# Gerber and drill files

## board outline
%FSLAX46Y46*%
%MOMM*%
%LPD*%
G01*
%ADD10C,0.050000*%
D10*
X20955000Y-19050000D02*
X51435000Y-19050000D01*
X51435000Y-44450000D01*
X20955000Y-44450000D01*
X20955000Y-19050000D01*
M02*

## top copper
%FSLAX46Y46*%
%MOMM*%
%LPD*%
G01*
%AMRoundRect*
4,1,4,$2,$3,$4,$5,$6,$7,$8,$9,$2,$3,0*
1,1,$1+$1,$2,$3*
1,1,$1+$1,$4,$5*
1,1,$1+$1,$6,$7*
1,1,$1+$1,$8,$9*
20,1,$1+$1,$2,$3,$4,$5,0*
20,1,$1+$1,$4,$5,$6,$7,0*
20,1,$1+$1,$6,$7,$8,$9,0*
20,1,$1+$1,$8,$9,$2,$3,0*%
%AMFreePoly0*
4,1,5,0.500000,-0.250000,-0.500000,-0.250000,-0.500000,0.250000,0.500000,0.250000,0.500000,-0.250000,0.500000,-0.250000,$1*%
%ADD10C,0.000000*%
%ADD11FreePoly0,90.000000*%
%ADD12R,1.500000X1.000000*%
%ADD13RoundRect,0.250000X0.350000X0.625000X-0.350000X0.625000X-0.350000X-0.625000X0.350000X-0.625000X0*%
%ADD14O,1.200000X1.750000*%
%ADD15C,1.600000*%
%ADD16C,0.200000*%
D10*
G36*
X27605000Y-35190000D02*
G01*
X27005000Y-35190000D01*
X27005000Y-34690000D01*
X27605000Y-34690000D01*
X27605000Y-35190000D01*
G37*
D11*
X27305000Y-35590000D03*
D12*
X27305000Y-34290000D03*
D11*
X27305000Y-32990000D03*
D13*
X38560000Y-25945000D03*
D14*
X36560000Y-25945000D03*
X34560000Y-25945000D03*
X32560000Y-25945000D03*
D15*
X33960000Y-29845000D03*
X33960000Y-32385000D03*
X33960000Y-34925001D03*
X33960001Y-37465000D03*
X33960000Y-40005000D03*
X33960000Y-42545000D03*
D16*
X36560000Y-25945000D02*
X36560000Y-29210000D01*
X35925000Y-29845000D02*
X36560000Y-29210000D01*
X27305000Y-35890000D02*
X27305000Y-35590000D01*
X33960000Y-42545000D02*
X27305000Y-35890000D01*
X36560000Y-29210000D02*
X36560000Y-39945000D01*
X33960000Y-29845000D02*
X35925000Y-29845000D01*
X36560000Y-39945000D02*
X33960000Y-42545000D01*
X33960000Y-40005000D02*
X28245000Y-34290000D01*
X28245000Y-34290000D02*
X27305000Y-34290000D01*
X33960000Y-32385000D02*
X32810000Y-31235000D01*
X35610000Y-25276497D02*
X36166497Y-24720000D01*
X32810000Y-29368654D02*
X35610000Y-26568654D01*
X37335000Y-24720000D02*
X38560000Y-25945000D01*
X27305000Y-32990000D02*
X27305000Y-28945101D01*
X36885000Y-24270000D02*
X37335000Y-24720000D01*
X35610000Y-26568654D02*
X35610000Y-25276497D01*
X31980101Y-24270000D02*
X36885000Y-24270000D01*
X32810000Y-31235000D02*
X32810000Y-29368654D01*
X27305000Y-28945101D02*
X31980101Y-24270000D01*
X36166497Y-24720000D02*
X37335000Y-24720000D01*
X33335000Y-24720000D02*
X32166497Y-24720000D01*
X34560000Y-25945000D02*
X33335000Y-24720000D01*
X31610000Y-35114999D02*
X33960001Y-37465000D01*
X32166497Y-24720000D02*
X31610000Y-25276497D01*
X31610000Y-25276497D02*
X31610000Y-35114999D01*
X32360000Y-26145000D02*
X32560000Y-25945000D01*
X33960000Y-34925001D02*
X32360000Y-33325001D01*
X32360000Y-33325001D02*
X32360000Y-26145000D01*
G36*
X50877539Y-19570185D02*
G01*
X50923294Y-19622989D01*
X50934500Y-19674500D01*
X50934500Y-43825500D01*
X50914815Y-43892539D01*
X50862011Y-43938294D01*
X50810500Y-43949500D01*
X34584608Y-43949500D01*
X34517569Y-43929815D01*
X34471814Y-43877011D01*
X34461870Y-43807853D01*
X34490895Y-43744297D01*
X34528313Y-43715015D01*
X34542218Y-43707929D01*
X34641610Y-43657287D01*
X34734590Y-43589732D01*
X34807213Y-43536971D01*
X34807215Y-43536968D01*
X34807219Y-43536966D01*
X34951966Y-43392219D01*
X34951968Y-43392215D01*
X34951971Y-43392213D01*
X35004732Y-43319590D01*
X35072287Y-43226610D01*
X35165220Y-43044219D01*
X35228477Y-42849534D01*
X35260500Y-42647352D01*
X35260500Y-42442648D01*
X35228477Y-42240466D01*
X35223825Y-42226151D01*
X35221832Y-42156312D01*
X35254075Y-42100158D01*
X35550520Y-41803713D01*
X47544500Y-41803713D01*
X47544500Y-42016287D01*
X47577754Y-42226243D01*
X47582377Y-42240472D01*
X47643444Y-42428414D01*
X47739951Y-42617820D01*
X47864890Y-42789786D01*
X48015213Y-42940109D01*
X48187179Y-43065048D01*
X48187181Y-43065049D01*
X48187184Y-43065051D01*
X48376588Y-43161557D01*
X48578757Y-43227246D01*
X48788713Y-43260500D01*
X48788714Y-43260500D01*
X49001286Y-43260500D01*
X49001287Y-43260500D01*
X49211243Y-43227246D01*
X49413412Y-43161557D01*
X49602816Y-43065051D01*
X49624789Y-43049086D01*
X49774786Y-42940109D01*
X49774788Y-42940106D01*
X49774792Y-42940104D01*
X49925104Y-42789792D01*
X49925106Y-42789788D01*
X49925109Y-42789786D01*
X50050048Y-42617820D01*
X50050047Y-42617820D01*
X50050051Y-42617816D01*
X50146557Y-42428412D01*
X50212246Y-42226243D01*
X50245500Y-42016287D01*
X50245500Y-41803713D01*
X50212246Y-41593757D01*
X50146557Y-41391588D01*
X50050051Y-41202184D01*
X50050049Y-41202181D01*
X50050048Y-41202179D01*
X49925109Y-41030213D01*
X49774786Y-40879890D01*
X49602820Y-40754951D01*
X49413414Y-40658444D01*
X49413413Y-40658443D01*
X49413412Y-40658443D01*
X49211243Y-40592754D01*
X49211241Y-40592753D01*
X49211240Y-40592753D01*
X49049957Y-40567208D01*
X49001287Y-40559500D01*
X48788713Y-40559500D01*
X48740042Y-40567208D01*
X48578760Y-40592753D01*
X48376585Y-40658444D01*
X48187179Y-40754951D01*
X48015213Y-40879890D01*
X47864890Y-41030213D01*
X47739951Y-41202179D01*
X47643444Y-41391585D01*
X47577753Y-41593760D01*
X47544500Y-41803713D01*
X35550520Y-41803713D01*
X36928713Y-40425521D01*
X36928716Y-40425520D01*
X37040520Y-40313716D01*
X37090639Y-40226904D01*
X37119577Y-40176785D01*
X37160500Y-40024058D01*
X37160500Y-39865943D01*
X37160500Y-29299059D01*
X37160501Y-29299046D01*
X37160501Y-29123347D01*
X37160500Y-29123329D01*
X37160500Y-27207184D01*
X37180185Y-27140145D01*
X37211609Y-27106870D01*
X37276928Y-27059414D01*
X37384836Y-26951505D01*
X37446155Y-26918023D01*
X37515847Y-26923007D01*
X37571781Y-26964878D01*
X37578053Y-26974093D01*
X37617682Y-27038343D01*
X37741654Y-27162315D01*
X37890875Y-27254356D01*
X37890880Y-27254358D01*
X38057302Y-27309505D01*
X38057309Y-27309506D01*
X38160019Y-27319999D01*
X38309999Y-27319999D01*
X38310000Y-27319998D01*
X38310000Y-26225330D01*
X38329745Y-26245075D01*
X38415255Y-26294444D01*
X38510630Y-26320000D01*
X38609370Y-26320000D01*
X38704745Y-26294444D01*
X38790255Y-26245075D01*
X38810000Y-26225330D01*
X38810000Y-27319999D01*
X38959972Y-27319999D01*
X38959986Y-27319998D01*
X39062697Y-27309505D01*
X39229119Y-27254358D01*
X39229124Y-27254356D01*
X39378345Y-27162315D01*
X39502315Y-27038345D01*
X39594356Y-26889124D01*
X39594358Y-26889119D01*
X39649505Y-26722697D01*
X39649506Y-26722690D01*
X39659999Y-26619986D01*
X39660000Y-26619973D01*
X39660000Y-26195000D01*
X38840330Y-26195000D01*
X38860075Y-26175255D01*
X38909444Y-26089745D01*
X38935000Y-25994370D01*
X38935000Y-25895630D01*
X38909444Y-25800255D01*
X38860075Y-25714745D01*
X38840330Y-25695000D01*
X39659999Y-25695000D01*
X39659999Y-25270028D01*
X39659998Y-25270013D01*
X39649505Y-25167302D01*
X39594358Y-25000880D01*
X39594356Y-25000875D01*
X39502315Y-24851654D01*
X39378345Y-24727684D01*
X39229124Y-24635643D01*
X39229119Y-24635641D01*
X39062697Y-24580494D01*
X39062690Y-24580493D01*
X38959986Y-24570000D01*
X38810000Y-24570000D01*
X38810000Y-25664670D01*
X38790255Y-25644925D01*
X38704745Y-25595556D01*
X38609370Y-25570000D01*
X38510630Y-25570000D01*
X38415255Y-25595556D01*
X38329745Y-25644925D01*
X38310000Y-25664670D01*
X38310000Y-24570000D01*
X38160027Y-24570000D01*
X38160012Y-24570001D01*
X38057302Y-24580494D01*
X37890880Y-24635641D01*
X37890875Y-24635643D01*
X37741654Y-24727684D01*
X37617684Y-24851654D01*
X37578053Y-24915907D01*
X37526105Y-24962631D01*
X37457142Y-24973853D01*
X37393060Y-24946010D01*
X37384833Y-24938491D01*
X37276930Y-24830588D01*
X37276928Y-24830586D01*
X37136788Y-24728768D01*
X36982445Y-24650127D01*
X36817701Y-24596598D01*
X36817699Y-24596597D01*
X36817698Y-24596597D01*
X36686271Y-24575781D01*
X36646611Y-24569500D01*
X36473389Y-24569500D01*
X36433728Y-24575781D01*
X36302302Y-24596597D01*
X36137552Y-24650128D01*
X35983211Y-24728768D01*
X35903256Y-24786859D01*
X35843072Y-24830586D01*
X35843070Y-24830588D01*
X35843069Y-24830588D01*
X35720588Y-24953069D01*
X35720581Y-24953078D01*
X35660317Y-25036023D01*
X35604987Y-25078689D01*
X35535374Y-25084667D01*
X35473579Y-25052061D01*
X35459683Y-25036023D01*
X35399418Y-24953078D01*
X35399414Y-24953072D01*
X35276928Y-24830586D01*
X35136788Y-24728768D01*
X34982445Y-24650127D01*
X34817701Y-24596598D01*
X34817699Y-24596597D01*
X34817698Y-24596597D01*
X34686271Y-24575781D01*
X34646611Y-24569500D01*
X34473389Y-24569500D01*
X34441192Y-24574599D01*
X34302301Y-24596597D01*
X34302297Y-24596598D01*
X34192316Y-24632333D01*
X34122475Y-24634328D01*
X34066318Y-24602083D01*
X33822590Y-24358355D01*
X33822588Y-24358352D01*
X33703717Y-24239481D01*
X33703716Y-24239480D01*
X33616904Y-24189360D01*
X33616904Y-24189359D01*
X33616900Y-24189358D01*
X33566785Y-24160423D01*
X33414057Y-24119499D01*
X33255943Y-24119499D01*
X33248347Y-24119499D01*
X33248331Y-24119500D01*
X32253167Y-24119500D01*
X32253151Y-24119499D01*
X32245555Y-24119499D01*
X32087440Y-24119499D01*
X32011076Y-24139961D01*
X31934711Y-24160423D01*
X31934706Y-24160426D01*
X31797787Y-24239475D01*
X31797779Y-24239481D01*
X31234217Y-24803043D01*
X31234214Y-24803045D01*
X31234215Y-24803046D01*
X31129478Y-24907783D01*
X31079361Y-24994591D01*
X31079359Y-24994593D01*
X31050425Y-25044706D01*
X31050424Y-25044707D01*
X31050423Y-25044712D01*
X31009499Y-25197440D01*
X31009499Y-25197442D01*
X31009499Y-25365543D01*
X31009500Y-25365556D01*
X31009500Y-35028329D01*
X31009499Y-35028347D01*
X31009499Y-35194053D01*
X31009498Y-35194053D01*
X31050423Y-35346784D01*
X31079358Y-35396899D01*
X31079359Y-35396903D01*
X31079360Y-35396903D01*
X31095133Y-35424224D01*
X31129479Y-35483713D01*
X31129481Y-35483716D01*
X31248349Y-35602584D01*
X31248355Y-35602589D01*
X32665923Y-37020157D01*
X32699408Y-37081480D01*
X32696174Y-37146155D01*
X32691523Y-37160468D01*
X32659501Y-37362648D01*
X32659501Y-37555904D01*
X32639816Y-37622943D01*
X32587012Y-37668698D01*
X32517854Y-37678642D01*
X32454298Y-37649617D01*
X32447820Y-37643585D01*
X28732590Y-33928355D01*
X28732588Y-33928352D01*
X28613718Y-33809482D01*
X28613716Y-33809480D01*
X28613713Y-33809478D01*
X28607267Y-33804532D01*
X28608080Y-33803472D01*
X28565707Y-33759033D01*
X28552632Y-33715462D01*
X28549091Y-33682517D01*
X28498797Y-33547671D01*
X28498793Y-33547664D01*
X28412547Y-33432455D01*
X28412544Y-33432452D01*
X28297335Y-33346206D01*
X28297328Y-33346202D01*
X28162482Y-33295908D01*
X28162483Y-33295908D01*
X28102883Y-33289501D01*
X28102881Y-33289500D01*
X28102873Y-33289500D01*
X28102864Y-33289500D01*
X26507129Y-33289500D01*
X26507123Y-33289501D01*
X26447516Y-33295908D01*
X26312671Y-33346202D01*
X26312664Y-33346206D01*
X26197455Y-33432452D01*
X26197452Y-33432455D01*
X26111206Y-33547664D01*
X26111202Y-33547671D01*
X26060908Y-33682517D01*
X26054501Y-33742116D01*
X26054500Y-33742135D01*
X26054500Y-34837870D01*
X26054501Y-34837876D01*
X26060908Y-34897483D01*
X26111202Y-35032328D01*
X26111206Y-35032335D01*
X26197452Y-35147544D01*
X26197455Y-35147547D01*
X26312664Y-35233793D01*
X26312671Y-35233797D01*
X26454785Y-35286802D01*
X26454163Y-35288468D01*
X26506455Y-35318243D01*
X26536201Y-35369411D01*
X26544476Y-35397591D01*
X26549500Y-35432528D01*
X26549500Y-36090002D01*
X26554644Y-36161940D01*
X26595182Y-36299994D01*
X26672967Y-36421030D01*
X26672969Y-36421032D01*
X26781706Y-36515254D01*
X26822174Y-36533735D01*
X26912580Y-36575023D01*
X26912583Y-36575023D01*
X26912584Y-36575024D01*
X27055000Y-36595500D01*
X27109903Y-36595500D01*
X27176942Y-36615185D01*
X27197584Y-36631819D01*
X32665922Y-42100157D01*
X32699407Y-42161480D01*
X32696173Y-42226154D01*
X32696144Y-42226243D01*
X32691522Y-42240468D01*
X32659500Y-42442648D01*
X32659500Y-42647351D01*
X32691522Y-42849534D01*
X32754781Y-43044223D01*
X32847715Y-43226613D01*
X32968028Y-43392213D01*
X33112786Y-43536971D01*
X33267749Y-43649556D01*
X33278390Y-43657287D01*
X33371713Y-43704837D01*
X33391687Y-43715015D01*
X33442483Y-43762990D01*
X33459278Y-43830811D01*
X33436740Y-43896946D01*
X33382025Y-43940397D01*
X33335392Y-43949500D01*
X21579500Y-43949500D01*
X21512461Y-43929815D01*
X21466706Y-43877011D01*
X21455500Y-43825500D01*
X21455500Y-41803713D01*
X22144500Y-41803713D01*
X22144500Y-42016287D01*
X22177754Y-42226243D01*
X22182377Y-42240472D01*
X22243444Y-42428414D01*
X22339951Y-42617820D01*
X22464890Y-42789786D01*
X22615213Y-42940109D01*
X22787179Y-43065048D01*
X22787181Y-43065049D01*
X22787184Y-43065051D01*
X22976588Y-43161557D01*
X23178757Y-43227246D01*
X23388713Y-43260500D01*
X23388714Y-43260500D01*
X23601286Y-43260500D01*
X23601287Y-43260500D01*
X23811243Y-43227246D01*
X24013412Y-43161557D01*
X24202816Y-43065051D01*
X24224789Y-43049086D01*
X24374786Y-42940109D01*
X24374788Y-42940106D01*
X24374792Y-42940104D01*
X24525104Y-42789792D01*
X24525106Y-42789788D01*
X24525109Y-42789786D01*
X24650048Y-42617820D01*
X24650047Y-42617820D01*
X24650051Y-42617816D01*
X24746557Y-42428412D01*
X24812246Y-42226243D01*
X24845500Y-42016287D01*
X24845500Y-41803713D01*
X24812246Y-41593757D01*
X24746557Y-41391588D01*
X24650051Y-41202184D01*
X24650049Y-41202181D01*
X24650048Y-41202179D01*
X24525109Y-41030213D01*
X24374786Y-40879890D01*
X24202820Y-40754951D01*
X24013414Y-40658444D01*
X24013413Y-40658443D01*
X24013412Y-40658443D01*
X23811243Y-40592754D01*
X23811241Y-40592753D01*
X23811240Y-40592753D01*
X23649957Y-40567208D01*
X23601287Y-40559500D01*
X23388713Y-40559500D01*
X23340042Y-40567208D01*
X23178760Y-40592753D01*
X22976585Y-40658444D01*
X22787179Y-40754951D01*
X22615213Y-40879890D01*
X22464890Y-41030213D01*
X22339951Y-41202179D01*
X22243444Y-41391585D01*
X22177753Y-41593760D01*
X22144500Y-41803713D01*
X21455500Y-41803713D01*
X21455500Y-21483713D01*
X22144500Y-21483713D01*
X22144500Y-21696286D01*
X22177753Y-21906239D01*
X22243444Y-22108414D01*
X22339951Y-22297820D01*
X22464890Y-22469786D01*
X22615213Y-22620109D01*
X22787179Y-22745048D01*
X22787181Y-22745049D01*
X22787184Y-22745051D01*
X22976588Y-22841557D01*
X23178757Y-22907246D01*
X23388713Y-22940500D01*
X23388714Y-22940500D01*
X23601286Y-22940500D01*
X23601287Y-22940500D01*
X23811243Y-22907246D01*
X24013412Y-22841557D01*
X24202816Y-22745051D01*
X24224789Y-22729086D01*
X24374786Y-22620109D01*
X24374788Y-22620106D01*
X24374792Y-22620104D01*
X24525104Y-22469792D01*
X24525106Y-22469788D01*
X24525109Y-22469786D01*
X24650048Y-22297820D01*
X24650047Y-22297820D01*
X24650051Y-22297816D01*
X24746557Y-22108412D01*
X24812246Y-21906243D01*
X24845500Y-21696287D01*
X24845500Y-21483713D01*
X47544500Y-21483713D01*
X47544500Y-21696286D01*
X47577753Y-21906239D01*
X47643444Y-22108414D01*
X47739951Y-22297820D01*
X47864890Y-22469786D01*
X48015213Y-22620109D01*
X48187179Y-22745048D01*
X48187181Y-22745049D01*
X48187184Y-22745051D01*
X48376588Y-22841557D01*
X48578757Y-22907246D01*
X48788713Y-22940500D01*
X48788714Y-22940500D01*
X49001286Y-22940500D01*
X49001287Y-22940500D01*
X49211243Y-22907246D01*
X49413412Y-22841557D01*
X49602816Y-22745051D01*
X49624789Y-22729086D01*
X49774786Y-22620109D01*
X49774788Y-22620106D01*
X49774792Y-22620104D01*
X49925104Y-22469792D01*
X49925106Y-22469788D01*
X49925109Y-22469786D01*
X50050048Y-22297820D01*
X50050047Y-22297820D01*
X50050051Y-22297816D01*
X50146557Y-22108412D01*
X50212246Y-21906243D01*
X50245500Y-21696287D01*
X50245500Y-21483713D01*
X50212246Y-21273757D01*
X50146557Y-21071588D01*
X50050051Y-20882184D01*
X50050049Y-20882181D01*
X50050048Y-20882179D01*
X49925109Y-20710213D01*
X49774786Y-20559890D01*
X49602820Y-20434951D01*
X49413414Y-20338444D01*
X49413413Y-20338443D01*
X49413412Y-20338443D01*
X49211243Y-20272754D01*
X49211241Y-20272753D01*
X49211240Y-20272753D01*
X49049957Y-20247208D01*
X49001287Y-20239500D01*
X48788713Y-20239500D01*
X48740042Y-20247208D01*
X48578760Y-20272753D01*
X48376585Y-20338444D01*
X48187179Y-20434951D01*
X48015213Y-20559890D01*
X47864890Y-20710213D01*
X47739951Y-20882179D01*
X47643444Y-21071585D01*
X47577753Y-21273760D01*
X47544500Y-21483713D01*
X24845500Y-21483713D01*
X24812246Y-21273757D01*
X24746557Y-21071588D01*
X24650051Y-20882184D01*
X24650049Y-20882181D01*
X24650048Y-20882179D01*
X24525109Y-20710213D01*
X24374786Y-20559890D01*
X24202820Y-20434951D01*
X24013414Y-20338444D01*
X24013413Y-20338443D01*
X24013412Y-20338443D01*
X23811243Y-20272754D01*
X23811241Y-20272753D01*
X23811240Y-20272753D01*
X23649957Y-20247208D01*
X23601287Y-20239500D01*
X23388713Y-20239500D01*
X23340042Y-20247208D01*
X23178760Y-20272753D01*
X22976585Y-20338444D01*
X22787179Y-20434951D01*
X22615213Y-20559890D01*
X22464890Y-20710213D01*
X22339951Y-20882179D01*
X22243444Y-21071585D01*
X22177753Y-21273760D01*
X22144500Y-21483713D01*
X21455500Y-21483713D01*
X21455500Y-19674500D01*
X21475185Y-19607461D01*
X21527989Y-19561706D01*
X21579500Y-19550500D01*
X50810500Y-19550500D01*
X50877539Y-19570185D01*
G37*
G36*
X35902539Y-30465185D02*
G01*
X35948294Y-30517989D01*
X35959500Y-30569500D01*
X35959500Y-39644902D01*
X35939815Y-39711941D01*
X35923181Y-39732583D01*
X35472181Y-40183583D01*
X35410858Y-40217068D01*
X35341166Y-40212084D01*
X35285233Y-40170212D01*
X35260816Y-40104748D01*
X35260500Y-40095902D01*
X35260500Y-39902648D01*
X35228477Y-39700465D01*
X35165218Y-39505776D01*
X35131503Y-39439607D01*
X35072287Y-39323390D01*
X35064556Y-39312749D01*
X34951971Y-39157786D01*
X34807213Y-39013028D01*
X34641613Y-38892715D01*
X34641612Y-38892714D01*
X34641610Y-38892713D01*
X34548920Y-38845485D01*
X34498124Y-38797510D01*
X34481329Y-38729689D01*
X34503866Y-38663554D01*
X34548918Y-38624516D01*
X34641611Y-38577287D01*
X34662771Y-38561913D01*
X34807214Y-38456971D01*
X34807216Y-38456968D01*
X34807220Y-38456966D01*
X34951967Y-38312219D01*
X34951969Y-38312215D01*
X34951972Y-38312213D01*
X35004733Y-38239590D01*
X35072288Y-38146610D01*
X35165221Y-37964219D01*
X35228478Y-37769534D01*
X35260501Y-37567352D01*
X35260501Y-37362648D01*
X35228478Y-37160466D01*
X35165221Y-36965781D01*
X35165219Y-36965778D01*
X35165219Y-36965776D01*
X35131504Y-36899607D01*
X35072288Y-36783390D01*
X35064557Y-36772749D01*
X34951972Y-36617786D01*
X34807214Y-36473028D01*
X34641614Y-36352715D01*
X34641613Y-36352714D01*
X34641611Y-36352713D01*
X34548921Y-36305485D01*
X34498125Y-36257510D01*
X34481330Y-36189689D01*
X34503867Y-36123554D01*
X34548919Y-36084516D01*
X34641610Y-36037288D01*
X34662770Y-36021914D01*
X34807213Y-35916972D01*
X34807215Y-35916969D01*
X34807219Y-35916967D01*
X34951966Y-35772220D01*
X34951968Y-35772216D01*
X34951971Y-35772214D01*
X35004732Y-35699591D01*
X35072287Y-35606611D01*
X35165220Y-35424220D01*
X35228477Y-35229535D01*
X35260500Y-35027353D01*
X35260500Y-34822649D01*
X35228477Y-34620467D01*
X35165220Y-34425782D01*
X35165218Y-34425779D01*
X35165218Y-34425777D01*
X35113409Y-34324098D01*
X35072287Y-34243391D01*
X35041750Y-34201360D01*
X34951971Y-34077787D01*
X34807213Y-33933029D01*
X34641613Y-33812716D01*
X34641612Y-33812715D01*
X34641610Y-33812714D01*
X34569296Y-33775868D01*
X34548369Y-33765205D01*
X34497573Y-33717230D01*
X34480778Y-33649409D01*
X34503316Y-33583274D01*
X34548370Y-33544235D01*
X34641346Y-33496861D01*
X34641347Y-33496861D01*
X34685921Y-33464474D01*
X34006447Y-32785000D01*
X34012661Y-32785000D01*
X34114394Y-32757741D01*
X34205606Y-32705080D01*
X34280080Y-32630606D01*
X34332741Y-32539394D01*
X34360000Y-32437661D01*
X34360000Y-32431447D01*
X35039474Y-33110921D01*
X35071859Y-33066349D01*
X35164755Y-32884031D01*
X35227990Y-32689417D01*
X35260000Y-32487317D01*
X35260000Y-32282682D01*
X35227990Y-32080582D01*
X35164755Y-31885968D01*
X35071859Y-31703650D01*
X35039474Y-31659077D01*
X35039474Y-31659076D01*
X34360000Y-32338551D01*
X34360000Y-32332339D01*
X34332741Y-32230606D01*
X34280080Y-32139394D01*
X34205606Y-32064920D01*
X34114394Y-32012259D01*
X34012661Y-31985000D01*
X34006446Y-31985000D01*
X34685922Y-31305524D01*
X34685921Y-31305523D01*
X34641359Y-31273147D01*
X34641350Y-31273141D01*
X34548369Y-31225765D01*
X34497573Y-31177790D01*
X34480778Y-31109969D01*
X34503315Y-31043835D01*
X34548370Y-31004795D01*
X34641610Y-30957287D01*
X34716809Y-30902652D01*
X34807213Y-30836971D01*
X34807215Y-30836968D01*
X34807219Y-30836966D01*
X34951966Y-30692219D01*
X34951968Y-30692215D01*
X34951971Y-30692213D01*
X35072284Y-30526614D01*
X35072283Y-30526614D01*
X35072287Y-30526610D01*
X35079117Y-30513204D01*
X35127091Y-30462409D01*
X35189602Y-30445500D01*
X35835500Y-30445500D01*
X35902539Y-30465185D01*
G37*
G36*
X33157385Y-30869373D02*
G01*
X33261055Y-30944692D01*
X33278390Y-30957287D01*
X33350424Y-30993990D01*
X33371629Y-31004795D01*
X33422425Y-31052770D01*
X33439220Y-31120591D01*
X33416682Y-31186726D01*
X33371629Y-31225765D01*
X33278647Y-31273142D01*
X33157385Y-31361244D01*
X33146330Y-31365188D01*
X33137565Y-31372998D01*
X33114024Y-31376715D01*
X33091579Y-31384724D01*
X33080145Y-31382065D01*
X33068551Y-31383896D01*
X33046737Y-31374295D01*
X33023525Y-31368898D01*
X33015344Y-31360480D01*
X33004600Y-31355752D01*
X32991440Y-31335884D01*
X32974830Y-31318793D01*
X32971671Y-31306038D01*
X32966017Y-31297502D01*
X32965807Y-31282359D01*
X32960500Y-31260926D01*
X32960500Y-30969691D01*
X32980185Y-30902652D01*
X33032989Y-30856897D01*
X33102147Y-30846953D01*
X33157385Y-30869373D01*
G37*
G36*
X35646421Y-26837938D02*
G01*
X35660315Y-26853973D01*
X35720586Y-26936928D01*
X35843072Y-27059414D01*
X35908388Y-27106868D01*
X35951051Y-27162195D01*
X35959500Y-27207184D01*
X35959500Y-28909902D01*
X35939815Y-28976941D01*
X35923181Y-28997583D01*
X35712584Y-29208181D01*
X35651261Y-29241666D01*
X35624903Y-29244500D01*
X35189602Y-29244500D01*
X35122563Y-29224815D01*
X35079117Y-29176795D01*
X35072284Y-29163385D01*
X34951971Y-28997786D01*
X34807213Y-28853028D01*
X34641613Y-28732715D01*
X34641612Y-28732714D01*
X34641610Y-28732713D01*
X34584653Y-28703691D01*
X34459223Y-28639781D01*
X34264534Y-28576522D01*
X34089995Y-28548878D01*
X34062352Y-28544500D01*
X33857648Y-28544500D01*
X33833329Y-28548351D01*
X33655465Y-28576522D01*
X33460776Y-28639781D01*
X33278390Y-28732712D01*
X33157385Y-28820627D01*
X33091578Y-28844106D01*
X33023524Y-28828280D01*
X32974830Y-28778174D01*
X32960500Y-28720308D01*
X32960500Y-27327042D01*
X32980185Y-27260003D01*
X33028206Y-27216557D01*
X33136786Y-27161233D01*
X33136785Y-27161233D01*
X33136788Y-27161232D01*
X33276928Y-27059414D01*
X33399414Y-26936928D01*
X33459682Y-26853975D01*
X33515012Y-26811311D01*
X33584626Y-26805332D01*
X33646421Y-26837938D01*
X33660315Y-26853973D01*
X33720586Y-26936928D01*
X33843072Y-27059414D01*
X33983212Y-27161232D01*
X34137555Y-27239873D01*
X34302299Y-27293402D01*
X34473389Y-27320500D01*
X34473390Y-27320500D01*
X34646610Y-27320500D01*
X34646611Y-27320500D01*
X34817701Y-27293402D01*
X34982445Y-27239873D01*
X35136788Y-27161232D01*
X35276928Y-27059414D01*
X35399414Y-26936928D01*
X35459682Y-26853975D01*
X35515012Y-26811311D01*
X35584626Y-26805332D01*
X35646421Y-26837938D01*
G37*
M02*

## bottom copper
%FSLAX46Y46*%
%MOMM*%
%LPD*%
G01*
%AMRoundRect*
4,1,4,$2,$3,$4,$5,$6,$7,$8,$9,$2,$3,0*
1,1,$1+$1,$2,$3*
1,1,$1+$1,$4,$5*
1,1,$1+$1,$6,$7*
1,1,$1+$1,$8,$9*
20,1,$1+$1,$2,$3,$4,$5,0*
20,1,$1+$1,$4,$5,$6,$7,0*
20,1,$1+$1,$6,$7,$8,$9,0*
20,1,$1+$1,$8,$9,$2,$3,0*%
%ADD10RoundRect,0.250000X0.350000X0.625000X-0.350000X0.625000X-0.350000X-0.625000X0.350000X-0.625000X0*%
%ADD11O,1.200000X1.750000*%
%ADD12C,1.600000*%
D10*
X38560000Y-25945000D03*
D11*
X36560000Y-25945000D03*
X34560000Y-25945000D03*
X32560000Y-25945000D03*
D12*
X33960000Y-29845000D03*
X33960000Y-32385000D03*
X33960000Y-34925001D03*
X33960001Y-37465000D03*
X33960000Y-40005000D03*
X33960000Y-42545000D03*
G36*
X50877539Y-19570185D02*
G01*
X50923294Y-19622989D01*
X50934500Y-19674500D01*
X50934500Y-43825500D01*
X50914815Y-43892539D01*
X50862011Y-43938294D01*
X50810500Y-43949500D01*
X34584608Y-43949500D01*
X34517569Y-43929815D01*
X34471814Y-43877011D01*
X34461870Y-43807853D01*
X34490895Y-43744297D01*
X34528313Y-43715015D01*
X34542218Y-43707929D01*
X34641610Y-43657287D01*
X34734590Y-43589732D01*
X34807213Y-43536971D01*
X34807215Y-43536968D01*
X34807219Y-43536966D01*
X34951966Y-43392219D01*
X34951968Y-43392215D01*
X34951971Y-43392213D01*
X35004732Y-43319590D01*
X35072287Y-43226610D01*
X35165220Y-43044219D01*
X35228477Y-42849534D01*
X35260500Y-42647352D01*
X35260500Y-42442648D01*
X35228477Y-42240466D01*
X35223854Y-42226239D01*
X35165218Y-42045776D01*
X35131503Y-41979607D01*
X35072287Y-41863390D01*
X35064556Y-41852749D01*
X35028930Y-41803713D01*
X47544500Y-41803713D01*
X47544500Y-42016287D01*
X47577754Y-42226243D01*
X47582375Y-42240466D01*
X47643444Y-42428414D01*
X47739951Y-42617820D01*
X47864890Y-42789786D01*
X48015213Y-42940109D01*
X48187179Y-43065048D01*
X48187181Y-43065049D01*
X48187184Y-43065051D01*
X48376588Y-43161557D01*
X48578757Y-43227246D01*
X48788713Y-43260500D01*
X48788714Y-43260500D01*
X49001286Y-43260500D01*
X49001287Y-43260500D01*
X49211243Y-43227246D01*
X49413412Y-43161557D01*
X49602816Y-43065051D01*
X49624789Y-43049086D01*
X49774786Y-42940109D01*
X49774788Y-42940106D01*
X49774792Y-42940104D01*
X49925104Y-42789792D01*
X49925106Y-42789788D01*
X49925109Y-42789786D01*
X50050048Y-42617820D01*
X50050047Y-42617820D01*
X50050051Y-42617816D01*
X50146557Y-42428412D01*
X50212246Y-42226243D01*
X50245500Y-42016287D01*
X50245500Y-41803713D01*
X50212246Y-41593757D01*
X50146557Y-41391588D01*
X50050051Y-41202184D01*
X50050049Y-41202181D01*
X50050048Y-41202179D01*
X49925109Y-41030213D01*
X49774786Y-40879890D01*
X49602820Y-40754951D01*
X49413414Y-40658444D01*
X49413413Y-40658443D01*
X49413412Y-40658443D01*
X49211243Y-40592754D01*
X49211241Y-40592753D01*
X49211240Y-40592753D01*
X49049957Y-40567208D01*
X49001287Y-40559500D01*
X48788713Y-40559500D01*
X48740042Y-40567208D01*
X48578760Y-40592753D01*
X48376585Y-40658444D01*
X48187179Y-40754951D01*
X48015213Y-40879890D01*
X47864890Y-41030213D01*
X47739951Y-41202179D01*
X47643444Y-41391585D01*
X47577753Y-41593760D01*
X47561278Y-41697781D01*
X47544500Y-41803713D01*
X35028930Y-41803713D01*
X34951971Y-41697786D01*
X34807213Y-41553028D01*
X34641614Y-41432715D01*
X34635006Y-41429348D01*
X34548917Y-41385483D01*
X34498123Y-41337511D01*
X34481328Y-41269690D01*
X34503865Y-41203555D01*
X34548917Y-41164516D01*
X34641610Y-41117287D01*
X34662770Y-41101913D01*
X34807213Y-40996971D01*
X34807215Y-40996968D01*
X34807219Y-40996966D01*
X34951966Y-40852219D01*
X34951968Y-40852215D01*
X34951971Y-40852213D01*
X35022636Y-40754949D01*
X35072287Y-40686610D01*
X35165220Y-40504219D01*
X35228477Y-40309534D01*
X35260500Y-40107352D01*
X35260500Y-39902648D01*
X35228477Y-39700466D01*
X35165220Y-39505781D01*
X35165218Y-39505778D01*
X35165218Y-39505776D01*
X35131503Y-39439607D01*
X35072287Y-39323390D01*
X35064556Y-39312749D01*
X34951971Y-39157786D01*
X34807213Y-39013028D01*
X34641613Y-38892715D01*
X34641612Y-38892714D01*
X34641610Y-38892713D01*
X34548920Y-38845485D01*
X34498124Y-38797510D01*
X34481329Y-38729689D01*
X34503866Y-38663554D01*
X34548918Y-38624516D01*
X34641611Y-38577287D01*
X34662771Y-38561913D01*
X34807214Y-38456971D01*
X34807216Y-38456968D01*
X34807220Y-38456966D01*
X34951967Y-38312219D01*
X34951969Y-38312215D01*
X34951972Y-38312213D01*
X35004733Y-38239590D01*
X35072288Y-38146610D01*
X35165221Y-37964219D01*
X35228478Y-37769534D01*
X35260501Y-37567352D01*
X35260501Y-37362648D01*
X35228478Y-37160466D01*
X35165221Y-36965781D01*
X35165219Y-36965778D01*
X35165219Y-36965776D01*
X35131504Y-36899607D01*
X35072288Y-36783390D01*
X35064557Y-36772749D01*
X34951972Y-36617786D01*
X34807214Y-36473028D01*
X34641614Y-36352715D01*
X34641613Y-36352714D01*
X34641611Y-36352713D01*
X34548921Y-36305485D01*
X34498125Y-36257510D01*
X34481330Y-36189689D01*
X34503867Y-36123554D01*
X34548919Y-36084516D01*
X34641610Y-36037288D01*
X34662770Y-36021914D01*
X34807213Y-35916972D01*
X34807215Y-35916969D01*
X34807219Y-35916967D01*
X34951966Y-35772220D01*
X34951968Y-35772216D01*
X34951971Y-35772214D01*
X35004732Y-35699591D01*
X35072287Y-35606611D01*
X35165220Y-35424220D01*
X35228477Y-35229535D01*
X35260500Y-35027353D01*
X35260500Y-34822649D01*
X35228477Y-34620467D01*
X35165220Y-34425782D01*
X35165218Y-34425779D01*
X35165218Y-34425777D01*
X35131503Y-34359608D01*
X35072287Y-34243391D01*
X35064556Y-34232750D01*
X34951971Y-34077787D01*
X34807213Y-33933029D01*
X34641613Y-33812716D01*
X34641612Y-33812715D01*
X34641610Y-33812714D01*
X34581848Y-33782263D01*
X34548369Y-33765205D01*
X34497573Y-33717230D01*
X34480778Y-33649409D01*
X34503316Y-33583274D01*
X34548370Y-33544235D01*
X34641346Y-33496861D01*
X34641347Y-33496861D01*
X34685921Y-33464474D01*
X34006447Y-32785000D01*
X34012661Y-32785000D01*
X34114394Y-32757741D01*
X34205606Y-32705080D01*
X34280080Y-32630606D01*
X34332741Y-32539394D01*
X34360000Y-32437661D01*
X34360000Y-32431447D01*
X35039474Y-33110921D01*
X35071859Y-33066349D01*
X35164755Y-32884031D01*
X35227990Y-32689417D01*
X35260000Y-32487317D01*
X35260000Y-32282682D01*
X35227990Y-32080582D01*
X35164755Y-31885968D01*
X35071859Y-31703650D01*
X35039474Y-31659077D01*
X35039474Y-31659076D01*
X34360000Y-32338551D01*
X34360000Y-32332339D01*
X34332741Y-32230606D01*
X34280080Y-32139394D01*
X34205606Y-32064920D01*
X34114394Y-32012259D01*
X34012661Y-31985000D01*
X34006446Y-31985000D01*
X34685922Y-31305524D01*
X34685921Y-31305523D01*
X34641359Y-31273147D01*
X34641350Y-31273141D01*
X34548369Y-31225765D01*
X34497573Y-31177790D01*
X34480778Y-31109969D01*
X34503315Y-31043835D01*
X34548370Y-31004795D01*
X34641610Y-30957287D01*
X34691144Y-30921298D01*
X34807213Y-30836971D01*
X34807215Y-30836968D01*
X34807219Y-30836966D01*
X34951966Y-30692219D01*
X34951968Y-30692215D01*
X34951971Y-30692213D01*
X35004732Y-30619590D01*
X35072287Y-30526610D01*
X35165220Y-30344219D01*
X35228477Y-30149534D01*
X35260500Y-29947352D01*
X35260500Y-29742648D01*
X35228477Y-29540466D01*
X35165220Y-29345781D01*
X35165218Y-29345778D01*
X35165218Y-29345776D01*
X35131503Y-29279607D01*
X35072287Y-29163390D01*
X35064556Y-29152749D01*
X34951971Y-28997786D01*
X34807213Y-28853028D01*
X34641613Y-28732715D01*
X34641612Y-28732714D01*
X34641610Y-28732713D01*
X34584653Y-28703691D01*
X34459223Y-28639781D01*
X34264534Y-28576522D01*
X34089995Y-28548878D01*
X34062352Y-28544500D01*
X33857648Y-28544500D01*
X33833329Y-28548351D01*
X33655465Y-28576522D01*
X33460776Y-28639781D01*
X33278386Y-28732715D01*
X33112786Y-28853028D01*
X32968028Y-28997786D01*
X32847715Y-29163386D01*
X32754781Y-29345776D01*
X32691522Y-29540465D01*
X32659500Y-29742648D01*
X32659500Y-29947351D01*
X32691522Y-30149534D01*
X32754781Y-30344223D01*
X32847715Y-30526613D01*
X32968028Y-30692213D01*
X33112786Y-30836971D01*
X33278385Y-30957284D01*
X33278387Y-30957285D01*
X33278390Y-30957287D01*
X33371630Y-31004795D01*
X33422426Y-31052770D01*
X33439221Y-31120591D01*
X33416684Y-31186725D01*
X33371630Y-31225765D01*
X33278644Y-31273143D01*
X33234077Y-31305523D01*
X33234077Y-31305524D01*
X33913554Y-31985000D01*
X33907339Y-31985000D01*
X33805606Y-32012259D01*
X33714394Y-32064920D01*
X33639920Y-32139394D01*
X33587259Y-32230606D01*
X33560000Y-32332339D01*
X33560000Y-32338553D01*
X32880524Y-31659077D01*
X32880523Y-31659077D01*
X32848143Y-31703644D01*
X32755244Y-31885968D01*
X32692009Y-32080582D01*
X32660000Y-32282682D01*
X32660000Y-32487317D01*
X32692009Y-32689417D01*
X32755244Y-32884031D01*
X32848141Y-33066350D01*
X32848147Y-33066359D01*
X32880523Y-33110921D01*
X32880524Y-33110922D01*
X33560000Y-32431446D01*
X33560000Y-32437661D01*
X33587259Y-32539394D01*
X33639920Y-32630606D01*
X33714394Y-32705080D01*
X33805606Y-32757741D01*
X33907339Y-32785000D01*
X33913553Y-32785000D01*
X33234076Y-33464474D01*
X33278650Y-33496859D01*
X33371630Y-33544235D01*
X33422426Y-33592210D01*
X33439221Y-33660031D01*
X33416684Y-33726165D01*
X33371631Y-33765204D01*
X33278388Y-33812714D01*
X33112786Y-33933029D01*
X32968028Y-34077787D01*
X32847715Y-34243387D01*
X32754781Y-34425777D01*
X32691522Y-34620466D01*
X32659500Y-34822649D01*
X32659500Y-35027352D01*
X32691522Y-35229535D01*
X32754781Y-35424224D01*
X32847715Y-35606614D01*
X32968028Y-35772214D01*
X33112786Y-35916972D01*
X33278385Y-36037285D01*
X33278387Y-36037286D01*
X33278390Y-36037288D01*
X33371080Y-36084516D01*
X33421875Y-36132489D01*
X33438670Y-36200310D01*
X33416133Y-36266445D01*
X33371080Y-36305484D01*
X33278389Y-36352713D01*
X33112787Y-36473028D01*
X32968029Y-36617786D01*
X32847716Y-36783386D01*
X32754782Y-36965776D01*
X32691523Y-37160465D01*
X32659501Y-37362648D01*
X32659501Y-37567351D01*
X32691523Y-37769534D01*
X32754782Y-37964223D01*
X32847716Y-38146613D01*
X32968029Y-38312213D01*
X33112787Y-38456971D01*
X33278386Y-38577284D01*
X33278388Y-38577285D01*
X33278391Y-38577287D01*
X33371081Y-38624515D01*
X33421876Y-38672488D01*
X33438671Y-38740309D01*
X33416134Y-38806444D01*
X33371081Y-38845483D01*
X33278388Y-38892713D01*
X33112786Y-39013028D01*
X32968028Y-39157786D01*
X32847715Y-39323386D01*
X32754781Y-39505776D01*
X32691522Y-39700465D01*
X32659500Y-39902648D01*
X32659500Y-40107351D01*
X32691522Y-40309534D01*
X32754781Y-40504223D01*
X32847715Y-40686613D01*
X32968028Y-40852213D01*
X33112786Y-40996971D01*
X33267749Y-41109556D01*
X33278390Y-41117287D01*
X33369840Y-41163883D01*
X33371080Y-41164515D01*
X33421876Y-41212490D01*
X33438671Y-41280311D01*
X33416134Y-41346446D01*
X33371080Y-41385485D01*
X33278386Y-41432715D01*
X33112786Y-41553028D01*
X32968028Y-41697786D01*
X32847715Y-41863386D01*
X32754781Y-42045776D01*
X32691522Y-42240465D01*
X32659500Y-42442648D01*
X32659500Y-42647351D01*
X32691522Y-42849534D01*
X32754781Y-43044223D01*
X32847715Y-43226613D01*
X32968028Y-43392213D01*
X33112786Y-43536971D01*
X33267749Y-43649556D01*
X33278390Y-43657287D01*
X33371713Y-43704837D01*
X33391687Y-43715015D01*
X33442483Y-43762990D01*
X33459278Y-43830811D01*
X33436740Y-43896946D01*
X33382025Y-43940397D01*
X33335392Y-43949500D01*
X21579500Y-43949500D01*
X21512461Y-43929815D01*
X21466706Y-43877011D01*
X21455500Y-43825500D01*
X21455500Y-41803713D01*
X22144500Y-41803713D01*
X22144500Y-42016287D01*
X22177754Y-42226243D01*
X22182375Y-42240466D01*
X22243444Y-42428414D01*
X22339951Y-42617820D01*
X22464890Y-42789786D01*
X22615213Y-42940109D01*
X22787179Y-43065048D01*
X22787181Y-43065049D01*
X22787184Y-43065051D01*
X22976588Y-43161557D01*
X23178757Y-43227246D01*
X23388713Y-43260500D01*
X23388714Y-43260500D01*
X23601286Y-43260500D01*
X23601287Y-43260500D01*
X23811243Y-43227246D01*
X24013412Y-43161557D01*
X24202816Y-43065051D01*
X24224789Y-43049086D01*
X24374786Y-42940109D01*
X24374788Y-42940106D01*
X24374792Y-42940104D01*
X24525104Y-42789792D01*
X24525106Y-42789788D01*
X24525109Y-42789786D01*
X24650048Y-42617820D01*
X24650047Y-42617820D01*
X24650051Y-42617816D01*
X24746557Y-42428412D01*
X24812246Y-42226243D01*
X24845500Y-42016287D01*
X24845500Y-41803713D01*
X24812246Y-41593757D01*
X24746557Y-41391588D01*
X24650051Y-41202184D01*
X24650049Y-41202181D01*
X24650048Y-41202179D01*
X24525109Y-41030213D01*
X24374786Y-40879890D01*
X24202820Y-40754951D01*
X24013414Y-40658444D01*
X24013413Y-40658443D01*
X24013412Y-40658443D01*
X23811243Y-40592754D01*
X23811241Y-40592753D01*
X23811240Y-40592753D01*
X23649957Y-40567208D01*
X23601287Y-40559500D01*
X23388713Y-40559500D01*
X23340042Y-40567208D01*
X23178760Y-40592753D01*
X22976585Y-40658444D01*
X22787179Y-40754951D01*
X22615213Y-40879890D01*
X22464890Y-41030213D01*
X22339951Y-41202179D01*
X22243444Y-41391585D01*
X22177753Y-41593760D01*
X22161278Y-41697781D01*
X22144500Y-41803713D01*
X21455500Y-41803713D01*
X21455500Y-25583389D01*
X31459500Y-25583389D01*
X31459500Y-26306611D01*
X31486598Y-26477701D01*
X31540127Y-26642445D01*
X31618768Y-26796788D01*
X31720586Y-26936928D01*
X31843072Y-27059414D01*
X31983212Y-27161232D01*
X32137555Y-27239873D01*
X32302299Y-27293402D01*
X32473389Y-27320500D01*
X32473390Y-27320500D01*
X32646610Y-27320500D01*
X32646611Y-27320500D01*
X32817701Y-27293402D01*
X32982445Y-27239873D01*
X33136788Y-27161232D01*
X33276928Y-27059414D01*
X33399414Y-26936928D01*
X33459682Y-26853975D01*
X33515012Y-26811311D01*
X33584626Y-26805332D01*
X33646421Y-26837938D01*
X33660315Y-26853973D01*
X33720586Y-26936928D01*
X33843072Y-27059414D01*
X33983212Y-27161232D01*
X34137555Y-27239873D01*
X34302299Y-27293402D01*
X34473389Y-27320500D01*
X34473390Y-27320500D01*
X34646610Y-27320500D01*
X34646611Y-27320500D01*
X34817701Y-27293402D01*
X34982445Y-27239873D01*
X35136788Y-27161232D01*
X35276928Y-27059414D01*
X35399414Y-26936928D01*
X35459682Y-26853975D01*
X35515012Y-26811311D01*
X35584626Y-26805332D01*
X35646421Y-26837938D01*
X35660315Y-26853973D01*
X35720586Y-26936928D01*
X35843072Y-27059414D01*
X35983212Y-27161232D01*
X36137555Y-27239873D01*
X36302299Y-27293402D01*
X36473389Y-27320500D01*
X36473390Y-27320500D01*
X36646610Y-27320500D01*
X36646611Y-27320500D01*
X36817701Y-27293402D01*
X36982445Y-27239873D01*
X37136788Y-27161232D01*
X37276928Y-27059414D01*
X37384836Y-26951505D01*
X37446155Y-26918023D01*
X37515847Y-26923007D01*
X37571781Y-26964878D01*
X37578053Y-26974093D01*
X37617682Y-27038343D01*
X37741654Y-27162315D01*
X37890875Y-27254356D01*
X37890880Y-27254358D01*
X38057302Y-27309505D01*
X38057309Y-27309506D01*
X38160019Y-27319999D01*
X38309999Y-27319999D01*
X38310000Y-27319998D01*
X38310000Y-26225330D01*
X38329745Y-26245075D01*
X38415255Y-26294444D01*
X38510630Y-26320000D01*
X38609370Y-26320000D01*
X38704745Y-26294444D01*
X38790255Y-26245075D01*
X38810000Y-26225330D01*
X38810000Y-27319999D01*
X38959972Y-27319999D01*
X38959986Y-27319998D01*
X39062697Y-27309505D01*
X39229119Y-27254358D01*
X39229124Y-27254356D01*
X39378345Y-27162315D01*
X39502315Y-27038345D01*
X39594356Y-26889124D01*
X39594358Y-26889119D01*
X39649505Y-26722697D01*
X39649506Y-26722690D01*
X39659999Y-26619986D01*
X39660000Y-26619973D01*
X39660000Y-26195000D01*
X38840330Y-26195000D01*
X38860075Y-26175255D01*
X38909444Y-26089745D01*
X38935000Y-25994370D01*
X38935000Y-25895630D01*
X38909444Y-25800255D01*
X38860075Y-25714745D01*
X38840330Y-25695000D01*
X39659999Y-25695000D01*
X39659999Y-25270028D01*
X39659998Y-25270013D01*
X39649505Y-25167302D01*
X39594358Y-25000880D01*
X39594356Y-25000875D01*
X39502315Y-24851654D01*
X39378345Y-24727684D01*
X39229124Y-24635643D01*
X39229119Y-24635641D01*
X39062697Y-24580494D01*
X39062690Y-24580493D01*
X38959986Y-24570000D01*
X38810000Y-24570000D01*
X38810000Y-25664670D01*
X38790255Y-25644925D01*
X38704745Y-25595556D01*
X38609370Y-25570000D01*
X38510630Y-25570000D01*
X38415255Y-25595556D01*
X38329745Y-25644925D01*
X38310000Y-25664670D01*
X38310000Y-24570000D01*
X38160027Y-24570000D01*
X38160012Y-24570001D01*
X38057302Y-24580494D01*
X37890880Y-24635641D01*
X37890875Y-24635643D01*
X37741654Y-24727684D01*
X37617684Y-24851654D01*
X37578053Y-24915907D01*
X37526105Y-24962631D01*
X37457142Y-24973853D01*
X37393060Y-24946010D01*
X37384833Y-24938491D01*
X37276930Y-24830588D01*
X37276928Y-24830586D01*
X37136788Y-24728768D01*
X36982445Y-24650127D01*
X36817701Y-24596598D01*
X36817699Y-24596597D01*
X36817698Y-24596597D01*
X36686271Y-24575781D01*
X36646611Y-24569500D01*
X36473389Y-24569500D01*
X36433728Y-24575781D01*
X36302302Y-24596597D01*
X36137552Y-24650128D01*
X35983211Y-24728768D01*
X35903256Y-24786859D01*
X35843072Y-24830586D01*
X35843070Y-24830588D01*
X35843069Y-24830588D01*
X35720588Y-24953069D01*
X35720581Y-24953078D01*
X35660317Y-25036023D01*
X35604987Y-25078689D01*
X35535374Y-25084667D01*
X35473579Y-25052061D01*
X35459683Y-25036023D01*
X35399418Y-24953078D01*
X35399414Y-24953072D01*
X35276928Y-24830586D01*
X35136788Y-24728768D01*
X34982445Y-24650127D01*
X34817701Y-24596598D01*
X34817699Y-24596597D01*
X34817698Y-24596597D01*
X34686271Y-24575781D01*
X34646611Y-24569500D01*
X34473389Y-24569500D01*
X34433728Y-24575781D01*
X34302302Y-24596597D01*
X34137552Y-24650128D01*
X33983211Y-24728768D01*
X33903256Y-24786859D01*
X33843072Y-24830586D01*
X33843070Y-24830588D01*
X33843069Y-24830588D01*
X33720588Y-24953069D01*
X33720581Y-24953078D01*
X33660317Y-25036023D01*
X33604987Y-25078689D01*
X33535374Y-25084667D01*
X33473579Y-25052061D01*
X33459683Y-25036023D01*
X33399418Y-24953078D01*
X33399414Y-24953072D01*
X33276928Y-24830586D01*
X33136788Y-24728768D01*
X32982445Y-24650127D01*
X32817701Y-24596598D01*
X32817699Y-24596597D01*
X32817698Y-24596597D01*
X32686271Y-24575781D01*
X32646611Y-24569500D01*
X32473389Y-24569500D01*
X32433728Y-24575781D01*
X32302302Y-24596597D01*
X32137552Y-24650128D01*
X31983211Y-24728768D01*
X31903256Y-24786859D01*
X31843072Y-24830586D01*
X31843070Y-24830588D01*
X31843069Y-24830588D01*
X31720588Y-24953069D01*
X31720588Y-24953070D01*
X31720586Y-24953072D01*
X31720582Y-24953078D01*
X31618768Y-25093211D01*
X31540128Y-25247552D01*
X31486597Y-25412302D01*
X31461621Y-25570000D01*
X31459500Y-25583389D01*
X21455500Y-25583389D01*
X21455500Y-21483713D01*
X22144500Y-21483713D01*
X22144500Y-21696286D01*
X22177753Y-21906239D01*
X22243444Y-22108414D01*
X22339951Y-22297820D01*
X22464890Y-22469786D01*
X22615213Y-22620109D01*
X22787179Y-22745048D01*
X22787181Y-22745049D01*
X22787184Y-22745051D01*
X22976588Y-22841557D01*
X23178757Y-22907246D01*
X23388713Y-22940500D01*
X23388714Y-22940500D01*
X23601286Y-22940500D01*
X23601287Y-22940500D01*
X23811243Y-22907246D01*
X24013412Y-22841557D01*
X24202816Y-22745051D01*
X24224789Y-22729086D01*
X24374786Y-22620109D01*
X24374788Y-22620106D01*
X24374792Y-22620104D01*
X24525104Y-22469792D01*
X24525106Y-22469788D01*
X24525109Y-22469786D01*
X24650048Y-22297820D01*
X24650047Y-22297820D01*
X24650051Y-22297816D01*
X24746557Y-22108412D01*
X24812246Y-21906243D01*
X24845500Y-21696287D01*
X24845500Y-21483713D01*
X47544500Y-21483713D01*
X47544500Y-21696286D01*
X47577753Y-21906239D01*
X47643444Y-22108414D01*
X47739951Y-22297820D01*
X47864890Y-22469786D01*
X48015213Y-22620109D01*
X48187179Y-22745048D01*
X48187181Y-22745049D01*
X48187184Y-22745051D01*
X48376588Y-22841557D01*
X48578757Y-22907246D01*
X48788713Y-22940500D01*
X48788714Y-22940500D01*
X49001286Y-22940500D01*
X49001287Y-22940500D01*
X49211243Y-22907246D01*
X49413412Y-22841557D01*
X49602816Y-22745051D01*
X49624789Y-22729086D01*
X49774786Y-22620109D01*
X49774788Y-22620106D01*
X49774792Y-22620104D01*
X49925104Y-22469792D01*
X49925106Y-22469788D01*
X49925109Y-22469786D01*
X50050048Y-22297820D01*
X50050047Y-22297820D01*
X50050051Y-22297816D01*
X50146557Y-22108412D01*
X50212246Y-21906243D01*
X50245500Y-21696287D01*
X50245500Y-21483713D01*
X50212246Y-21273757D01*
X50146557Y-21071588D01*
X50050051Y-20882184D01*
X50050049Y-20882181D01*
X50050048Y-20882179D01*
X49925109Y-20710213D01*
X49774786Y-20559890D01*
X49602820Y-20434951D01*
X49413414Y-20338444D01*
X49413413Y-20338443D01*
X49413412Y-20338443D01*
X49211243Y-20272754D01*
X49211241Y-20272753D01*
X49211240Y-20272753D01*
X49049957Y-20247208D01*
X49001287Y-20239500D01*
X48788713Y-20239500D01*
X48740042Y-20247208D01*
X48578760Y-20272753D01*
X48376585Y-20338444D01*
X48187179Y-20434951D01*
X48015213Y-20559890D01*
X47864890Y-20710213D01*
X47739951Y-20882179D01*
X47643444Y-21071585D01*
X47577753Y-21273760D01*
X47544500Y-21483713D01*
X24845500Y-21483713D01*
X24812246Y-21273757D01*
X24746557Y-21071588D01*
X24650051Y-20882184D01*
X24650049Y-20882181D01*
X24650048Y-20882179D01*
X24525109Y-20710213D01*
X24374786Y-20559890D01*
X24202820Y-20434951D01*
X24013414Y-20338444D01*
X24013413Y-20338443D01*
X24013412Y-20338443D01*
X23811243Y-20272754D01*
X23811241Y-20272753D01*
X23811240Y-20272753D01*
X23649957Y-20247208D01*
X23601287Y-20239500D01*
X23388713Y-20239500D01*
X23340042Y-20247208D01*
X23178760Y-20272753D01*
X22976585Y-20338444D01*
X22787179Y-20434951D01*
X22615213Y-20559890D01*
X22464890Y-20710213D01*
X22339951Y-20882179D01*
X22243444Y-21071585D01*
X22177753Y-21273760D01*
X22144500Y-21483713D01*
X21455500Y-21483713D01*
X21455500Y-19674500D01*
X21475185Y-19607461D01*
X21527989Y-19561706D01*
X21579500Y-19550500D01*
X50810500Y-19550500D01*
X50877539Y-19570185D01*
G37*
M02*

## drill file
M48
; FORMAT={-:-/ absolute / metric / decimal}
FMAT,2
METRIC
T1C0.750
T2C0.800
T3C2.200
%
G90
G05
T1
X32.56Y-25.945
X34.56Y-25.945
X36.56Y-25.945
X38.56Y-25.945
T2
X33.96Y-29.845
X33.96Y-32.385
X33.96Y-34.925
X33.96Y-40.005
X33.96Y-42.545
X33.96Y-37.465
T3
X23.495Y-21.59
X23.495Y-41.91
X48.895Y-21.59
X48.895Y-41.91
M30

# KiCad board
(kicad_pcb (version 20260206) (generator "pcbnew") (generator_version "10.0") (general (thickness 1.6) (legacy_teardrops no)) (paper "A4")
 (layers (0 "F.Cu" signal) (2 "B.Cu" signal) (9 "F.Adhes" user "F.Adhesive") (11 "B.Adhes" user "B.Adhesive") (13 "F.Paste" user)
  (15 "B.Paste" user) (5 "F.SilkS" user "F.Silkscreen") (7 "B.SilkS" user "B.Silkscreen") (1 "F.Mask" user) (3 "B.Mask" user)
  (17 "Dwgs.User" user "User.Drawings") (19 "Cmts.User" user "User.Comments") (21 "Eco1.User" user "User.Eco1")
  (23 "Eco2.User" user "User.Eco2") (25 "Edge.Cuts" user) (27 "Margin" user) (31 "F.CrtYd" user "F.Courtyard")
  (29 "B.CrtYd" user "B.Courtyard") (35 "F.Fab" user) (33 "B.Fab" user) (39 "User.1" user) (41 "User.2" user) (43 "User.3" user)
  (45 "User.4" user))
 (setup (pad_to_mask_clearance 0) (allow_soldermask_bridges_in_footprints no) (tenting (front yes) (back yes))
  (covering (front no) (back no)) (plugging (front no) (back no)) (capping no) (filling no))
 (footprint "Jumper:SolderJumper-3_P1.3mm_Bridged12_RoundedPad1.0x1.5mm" (layer "F.Cu") (at 27.305 34.29 90)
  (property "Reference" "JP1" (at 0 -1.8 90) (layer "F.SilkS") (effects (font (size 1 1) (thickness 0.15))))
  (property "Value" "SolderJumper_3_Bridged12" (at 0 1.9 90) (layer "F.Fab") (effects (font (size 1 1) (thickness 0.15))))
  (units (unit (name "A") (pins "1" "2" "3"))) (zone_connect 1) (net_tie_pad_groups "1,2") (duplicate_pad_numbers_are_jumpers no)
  (fp_poly (pts (xy -0.9 -0.3) (xy -0.4 -0.3) (xy -0.4 0.3) (xy -0.9 0.3)) (stroke (width 0) (type solid)) (fill yes) (layer "F.Cu"))
  (pad "1" smd custom (at -1.3 0 90) (size 1 0.5) (layers "F.Cu" "F.Mask") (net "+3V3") (zone_connect 2) (thermal_bridge_angle 45)
   (options (clearance outline) (anchor rect)) (primitives))
  (pad "2" smd rect (at 0 0 90) (size 1 1.5) (layers "F.Cu" "F.Mask") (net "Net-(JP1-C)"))
  (pad "3" smd custom (at 1.3 0 90) (size 1 0.5) (layers "F.Cu" "F.Mask") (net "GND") (zone_connect 2) (thermal_bridge_angle 45)
   (options (clearance outline) (anchor rect)) (primitives)))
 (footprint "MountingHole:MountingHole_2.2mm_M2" (layer "F.Cu") (at 48.895 21.59)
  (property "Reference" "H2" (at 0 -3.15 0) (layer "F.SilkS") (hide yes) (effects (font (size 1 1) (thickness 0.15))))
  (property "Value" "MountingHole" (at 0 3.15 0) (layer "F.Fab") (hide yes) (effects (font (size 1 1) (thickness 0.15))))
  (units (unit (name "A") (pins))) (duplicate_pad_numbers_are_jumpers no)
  (pad "" np_thru_hole circle (at 0 0) (size 2.2 2.2) (drill 2.2) (layers "*.Cu" "*.Mask")))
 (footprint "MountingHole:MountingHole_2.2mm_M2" (layer "F.Cu") (at 48.895 41.91)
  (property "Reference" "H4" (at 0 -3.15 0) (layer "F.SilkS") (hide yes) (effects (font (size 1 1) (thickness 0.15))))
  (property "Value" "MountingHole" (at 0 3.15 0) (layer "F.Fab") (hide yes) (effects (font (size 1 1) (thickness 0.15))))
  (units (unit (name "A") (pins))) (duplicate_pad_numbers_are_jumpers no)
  (pad "" np_thru_hole circle (at 0 0) (size 2.2 2.2) (drill 2.2) (layers "*.Cu" "*.Mask")))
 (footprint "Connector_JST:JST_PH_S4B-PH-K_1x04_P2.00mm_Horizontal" (layer "F.Cu") (at 38.56 25.945 180)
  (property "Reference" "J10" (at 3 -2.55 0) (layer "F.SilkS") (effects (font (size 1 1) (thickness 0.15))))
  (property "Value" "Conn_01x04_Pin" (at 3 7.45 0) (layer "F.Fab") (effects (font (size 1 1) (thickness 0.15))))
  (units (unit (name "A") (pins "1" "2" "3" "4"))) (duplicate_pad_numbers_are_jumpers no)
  (pad "1" thru_hole roundrect (at 0 0 180) (size 1.2 1.75) (drill 0.75) (layers "*.Cu" "*.Mask") (remove_unused_layers no)
   (roundrect_rratio 0.208333) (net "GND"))
  (pad "2" thru_hole oval (at 2 0 180) (size 1.2 1.75) (drill 0.75) (layers "*.Cu" "*.Mask") (remove_unused_layers no) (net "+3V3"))
  (pad "3" thru_hole oval (at 4 0 180) (size 1.2 1.75) (drill 0.75) (layers "*.Cu" "*.Mask") (remove_unused_layers no) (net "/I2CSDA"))
  (pad "4" thru_hole oval (at 6 0 180) (size 1.2 1.75) (drill 0.75) (layers "*.Cu" "*.Mask") (remove_unused_layers no) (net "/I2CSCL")))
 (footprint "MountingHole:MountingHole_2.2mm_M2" (layer "F.Cu") (at 23.495 21.59)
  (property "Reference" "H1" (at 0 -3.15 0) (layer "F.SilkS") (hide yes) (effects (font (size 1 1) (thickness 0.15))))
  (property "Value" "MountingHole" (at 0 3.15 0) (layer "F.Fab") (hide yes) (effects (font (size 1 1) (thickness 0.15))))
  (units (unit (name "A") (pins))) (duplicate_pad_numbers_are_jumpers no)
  (pad "" np_thru_hole circle (at 0 0) (size 2.2 2.2) (drill 2.2) (layers "*.Cu" "*.Mask")))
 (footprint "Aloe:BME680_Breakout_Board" (layer "F.Cu") (at 40.31 36.195 -90)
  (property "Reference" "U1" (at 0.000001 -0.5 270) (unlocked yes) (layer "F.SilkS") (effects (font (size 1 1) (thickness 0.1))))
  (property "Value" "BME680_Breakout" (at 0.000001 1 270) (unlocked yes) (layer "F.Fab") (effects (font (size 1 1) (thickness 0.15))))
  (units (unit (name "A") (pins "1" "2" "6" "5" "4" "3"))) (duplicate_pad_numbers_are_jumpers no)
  (pad "1" thru_hole circle (at -6.35 6.35 270) (size 1.6 1.6) (drill 0.8) (layers "*.Cu" "*.Mask") (remove_unused_layers no) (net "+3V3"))
  (pad "2" thru_hole circle (at -3.81 6.35 270) (size 1.6 1.6) (drill 0.8) (layers "*.Cu" "*.Mask") (remove_unused_layers no) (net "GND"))
  (pad "3" thru_hole circle (at -1.269999 6.35 270) (size 1.6 1.6) (drill 0.8) (layers "*.Cu" "*.Mask") (remove_unused_layers no)
   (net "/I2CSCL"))
  (pad "4" thru_hole circle (at 1.27 6.349999 270) (size 1.6 1.6) (drill 0.8) (layers "*.Cu" "*.Mask") (remove_unused_layers no)
   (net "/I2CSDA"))
  (pad "5" thru_hole circle (at 3.81 6.35 270) (size 1.6 1.6) (drill 0.8) (layers "*.Cu" "*.Mask") (remove_unused_layers no)
   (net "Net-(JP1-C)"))
  (pad "6" thru_hole circle (at 6.35 6.35 270) (size 1.6 1.6) (drill 0.8) (layers "*.Cu" "*.Mask") (remove_unused_layers no) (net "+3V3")))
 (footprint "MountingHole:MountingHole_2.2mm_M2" (layer "F.Cu") (at 23.495 41.91)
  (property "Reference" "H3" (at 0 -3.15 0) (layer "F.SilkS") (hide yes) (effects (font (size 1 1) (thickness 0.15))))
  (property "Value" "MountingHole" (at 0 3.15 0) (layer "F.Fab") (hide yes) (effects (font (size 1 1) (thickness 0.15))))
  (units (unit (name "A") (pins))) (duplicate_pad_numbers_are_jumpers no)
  (pad "" np_thru_hole circle (at 0 0) (size 2.2 2.2) (drill 2.2) (layers "*.Cu" "*.Mask")))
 (gr_rect (start 20.955 19.05) (end 51.435 44.45) (stroke (width 0.05) (type solid)) (fill no) (layer "Edge.Cuts"))
 (segment (start 36.56 25.945) (end 36.56 29.21) (width 0.2) (layer "F.Cu") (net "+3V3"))
 (segment (start 35.925 29.845) (end 36.56 29.21) (width 0.2) (layer "F.Cu") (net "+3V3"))
 (segment (start 27.305 35.89) (end 27.305 35.59) (width 0.2) (layer "F.Cu") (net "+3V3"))
 (segment (start 33.96 42.545) (end 27.305 35.89) (width 0.2) (layer "F.Cu") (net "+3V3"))
 (segment (start 36.56 29.21) (end 36.56 39.945) (width 0.2) (layer "F.Cu") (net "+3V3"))
 (segment (start 33.96 29.845) (end 35.925 29.845) (width 0.2) (layer "F.Cu") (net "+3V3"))
 (segment (start 36.56 39.945) (end 33.96 42.545) (width 0.2) (layer "F.Cu") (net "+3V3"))
 (segment (start 33.96 40.005) (end 28.245 34.29) (width 0.2) (layer "F.Cu") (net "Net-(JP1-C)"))
 (segment (start 28.245 34.29) (end 27.305 34.29) (width 0.2) (layer "F.Cu") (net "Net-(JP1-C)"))
 (segment (start 33.96 32.385) (end 32.81 31.235) (width 0.2) (layer "F.Cu") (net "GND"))
 (segment (start 35.61 25.276497) (end 36.166497 24.72) (width 0.2) (layer "F.Cu") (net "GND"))
 (segment (start 32.81 29.368654) (end 35.61 26.568654) (width 0.2) (layer "F.Cu") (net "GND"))
 (segment (start 37.335 24.72) (end 38.56 25.945) (width 0.2) (layer "F.Cu") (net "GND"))
 (segment (start 27.305 32.99) (end 27.305 28.945101) (width 0.2) (layer "F.Cu") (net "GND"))
 (segment (start 36.885 24.27) (end 37.335 24.72) (width 0.2) (layer "F.Cu") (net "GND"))
 (segment (start 35.61 26.568654) (end 35.61 25.276497) (width 0.2) (layer "F.Cu") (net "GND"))
 (segment (start 31.980101 24.27) (end 36.885 24.27) (width 0.2) (layer "F.Cu") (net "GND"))
 (segment (start 32.81 31.235) (end 32.81 29.368654) (width 0.2) (layer "F.Cu") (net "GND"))
 (segment (start 27.305 28.945101) (end 31.980101 24.27) (width 0.2) (layer "F.Cu") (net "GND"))
 (segment (start 36.166497 24.72) (end 37.335 24.72) (width 0.2) (layer "F.Cu") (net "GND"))
 (segment (start 33.335 24.72) (end 32.166497 24.72) (width 0.2) (layer "F.Cu") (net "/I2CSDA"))
 (segment (start 34.56 25.945) (end 33.335 24.72) (width 0.2) (layer "F.Cu") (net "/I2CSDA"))
 (segment (start 31.61 35.114999) (end 33.960001 37.465) (width 0.2) (layer "F.Cu") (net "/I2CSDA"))
 (segment (start 32.166497 24.72) (end 31.61 25.276497) (width 0.2) (layer "F.Cu") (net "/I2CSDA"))
 (segment (start 31.61 25.276497) (end 31.61 35.114999) (width 0.2) (layer "F.Cu") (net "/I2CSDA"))
 (segment (start 32.36 26.145) (end 32.56 25.945) (width 0.2) (layer "F.Cu") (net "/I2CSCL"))
 (segment (start 33.96 34.925001) (end 32.36 33.325001) (width 0.2) (layer "F.Cu") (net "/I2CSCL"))
 (segment (start 32.36 33.325001) (end 32.36 26.145) (width 0.2) (layer "F.Cu") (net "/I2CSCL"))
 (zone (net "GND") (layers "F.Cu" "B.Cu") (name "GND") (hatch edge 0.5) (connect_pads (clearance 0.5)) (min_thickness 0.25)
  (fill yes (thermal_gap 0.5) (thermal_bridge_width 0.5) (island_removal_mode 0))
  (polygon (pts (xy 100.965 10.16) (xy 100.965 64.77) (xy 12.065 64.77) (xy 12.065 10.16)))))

